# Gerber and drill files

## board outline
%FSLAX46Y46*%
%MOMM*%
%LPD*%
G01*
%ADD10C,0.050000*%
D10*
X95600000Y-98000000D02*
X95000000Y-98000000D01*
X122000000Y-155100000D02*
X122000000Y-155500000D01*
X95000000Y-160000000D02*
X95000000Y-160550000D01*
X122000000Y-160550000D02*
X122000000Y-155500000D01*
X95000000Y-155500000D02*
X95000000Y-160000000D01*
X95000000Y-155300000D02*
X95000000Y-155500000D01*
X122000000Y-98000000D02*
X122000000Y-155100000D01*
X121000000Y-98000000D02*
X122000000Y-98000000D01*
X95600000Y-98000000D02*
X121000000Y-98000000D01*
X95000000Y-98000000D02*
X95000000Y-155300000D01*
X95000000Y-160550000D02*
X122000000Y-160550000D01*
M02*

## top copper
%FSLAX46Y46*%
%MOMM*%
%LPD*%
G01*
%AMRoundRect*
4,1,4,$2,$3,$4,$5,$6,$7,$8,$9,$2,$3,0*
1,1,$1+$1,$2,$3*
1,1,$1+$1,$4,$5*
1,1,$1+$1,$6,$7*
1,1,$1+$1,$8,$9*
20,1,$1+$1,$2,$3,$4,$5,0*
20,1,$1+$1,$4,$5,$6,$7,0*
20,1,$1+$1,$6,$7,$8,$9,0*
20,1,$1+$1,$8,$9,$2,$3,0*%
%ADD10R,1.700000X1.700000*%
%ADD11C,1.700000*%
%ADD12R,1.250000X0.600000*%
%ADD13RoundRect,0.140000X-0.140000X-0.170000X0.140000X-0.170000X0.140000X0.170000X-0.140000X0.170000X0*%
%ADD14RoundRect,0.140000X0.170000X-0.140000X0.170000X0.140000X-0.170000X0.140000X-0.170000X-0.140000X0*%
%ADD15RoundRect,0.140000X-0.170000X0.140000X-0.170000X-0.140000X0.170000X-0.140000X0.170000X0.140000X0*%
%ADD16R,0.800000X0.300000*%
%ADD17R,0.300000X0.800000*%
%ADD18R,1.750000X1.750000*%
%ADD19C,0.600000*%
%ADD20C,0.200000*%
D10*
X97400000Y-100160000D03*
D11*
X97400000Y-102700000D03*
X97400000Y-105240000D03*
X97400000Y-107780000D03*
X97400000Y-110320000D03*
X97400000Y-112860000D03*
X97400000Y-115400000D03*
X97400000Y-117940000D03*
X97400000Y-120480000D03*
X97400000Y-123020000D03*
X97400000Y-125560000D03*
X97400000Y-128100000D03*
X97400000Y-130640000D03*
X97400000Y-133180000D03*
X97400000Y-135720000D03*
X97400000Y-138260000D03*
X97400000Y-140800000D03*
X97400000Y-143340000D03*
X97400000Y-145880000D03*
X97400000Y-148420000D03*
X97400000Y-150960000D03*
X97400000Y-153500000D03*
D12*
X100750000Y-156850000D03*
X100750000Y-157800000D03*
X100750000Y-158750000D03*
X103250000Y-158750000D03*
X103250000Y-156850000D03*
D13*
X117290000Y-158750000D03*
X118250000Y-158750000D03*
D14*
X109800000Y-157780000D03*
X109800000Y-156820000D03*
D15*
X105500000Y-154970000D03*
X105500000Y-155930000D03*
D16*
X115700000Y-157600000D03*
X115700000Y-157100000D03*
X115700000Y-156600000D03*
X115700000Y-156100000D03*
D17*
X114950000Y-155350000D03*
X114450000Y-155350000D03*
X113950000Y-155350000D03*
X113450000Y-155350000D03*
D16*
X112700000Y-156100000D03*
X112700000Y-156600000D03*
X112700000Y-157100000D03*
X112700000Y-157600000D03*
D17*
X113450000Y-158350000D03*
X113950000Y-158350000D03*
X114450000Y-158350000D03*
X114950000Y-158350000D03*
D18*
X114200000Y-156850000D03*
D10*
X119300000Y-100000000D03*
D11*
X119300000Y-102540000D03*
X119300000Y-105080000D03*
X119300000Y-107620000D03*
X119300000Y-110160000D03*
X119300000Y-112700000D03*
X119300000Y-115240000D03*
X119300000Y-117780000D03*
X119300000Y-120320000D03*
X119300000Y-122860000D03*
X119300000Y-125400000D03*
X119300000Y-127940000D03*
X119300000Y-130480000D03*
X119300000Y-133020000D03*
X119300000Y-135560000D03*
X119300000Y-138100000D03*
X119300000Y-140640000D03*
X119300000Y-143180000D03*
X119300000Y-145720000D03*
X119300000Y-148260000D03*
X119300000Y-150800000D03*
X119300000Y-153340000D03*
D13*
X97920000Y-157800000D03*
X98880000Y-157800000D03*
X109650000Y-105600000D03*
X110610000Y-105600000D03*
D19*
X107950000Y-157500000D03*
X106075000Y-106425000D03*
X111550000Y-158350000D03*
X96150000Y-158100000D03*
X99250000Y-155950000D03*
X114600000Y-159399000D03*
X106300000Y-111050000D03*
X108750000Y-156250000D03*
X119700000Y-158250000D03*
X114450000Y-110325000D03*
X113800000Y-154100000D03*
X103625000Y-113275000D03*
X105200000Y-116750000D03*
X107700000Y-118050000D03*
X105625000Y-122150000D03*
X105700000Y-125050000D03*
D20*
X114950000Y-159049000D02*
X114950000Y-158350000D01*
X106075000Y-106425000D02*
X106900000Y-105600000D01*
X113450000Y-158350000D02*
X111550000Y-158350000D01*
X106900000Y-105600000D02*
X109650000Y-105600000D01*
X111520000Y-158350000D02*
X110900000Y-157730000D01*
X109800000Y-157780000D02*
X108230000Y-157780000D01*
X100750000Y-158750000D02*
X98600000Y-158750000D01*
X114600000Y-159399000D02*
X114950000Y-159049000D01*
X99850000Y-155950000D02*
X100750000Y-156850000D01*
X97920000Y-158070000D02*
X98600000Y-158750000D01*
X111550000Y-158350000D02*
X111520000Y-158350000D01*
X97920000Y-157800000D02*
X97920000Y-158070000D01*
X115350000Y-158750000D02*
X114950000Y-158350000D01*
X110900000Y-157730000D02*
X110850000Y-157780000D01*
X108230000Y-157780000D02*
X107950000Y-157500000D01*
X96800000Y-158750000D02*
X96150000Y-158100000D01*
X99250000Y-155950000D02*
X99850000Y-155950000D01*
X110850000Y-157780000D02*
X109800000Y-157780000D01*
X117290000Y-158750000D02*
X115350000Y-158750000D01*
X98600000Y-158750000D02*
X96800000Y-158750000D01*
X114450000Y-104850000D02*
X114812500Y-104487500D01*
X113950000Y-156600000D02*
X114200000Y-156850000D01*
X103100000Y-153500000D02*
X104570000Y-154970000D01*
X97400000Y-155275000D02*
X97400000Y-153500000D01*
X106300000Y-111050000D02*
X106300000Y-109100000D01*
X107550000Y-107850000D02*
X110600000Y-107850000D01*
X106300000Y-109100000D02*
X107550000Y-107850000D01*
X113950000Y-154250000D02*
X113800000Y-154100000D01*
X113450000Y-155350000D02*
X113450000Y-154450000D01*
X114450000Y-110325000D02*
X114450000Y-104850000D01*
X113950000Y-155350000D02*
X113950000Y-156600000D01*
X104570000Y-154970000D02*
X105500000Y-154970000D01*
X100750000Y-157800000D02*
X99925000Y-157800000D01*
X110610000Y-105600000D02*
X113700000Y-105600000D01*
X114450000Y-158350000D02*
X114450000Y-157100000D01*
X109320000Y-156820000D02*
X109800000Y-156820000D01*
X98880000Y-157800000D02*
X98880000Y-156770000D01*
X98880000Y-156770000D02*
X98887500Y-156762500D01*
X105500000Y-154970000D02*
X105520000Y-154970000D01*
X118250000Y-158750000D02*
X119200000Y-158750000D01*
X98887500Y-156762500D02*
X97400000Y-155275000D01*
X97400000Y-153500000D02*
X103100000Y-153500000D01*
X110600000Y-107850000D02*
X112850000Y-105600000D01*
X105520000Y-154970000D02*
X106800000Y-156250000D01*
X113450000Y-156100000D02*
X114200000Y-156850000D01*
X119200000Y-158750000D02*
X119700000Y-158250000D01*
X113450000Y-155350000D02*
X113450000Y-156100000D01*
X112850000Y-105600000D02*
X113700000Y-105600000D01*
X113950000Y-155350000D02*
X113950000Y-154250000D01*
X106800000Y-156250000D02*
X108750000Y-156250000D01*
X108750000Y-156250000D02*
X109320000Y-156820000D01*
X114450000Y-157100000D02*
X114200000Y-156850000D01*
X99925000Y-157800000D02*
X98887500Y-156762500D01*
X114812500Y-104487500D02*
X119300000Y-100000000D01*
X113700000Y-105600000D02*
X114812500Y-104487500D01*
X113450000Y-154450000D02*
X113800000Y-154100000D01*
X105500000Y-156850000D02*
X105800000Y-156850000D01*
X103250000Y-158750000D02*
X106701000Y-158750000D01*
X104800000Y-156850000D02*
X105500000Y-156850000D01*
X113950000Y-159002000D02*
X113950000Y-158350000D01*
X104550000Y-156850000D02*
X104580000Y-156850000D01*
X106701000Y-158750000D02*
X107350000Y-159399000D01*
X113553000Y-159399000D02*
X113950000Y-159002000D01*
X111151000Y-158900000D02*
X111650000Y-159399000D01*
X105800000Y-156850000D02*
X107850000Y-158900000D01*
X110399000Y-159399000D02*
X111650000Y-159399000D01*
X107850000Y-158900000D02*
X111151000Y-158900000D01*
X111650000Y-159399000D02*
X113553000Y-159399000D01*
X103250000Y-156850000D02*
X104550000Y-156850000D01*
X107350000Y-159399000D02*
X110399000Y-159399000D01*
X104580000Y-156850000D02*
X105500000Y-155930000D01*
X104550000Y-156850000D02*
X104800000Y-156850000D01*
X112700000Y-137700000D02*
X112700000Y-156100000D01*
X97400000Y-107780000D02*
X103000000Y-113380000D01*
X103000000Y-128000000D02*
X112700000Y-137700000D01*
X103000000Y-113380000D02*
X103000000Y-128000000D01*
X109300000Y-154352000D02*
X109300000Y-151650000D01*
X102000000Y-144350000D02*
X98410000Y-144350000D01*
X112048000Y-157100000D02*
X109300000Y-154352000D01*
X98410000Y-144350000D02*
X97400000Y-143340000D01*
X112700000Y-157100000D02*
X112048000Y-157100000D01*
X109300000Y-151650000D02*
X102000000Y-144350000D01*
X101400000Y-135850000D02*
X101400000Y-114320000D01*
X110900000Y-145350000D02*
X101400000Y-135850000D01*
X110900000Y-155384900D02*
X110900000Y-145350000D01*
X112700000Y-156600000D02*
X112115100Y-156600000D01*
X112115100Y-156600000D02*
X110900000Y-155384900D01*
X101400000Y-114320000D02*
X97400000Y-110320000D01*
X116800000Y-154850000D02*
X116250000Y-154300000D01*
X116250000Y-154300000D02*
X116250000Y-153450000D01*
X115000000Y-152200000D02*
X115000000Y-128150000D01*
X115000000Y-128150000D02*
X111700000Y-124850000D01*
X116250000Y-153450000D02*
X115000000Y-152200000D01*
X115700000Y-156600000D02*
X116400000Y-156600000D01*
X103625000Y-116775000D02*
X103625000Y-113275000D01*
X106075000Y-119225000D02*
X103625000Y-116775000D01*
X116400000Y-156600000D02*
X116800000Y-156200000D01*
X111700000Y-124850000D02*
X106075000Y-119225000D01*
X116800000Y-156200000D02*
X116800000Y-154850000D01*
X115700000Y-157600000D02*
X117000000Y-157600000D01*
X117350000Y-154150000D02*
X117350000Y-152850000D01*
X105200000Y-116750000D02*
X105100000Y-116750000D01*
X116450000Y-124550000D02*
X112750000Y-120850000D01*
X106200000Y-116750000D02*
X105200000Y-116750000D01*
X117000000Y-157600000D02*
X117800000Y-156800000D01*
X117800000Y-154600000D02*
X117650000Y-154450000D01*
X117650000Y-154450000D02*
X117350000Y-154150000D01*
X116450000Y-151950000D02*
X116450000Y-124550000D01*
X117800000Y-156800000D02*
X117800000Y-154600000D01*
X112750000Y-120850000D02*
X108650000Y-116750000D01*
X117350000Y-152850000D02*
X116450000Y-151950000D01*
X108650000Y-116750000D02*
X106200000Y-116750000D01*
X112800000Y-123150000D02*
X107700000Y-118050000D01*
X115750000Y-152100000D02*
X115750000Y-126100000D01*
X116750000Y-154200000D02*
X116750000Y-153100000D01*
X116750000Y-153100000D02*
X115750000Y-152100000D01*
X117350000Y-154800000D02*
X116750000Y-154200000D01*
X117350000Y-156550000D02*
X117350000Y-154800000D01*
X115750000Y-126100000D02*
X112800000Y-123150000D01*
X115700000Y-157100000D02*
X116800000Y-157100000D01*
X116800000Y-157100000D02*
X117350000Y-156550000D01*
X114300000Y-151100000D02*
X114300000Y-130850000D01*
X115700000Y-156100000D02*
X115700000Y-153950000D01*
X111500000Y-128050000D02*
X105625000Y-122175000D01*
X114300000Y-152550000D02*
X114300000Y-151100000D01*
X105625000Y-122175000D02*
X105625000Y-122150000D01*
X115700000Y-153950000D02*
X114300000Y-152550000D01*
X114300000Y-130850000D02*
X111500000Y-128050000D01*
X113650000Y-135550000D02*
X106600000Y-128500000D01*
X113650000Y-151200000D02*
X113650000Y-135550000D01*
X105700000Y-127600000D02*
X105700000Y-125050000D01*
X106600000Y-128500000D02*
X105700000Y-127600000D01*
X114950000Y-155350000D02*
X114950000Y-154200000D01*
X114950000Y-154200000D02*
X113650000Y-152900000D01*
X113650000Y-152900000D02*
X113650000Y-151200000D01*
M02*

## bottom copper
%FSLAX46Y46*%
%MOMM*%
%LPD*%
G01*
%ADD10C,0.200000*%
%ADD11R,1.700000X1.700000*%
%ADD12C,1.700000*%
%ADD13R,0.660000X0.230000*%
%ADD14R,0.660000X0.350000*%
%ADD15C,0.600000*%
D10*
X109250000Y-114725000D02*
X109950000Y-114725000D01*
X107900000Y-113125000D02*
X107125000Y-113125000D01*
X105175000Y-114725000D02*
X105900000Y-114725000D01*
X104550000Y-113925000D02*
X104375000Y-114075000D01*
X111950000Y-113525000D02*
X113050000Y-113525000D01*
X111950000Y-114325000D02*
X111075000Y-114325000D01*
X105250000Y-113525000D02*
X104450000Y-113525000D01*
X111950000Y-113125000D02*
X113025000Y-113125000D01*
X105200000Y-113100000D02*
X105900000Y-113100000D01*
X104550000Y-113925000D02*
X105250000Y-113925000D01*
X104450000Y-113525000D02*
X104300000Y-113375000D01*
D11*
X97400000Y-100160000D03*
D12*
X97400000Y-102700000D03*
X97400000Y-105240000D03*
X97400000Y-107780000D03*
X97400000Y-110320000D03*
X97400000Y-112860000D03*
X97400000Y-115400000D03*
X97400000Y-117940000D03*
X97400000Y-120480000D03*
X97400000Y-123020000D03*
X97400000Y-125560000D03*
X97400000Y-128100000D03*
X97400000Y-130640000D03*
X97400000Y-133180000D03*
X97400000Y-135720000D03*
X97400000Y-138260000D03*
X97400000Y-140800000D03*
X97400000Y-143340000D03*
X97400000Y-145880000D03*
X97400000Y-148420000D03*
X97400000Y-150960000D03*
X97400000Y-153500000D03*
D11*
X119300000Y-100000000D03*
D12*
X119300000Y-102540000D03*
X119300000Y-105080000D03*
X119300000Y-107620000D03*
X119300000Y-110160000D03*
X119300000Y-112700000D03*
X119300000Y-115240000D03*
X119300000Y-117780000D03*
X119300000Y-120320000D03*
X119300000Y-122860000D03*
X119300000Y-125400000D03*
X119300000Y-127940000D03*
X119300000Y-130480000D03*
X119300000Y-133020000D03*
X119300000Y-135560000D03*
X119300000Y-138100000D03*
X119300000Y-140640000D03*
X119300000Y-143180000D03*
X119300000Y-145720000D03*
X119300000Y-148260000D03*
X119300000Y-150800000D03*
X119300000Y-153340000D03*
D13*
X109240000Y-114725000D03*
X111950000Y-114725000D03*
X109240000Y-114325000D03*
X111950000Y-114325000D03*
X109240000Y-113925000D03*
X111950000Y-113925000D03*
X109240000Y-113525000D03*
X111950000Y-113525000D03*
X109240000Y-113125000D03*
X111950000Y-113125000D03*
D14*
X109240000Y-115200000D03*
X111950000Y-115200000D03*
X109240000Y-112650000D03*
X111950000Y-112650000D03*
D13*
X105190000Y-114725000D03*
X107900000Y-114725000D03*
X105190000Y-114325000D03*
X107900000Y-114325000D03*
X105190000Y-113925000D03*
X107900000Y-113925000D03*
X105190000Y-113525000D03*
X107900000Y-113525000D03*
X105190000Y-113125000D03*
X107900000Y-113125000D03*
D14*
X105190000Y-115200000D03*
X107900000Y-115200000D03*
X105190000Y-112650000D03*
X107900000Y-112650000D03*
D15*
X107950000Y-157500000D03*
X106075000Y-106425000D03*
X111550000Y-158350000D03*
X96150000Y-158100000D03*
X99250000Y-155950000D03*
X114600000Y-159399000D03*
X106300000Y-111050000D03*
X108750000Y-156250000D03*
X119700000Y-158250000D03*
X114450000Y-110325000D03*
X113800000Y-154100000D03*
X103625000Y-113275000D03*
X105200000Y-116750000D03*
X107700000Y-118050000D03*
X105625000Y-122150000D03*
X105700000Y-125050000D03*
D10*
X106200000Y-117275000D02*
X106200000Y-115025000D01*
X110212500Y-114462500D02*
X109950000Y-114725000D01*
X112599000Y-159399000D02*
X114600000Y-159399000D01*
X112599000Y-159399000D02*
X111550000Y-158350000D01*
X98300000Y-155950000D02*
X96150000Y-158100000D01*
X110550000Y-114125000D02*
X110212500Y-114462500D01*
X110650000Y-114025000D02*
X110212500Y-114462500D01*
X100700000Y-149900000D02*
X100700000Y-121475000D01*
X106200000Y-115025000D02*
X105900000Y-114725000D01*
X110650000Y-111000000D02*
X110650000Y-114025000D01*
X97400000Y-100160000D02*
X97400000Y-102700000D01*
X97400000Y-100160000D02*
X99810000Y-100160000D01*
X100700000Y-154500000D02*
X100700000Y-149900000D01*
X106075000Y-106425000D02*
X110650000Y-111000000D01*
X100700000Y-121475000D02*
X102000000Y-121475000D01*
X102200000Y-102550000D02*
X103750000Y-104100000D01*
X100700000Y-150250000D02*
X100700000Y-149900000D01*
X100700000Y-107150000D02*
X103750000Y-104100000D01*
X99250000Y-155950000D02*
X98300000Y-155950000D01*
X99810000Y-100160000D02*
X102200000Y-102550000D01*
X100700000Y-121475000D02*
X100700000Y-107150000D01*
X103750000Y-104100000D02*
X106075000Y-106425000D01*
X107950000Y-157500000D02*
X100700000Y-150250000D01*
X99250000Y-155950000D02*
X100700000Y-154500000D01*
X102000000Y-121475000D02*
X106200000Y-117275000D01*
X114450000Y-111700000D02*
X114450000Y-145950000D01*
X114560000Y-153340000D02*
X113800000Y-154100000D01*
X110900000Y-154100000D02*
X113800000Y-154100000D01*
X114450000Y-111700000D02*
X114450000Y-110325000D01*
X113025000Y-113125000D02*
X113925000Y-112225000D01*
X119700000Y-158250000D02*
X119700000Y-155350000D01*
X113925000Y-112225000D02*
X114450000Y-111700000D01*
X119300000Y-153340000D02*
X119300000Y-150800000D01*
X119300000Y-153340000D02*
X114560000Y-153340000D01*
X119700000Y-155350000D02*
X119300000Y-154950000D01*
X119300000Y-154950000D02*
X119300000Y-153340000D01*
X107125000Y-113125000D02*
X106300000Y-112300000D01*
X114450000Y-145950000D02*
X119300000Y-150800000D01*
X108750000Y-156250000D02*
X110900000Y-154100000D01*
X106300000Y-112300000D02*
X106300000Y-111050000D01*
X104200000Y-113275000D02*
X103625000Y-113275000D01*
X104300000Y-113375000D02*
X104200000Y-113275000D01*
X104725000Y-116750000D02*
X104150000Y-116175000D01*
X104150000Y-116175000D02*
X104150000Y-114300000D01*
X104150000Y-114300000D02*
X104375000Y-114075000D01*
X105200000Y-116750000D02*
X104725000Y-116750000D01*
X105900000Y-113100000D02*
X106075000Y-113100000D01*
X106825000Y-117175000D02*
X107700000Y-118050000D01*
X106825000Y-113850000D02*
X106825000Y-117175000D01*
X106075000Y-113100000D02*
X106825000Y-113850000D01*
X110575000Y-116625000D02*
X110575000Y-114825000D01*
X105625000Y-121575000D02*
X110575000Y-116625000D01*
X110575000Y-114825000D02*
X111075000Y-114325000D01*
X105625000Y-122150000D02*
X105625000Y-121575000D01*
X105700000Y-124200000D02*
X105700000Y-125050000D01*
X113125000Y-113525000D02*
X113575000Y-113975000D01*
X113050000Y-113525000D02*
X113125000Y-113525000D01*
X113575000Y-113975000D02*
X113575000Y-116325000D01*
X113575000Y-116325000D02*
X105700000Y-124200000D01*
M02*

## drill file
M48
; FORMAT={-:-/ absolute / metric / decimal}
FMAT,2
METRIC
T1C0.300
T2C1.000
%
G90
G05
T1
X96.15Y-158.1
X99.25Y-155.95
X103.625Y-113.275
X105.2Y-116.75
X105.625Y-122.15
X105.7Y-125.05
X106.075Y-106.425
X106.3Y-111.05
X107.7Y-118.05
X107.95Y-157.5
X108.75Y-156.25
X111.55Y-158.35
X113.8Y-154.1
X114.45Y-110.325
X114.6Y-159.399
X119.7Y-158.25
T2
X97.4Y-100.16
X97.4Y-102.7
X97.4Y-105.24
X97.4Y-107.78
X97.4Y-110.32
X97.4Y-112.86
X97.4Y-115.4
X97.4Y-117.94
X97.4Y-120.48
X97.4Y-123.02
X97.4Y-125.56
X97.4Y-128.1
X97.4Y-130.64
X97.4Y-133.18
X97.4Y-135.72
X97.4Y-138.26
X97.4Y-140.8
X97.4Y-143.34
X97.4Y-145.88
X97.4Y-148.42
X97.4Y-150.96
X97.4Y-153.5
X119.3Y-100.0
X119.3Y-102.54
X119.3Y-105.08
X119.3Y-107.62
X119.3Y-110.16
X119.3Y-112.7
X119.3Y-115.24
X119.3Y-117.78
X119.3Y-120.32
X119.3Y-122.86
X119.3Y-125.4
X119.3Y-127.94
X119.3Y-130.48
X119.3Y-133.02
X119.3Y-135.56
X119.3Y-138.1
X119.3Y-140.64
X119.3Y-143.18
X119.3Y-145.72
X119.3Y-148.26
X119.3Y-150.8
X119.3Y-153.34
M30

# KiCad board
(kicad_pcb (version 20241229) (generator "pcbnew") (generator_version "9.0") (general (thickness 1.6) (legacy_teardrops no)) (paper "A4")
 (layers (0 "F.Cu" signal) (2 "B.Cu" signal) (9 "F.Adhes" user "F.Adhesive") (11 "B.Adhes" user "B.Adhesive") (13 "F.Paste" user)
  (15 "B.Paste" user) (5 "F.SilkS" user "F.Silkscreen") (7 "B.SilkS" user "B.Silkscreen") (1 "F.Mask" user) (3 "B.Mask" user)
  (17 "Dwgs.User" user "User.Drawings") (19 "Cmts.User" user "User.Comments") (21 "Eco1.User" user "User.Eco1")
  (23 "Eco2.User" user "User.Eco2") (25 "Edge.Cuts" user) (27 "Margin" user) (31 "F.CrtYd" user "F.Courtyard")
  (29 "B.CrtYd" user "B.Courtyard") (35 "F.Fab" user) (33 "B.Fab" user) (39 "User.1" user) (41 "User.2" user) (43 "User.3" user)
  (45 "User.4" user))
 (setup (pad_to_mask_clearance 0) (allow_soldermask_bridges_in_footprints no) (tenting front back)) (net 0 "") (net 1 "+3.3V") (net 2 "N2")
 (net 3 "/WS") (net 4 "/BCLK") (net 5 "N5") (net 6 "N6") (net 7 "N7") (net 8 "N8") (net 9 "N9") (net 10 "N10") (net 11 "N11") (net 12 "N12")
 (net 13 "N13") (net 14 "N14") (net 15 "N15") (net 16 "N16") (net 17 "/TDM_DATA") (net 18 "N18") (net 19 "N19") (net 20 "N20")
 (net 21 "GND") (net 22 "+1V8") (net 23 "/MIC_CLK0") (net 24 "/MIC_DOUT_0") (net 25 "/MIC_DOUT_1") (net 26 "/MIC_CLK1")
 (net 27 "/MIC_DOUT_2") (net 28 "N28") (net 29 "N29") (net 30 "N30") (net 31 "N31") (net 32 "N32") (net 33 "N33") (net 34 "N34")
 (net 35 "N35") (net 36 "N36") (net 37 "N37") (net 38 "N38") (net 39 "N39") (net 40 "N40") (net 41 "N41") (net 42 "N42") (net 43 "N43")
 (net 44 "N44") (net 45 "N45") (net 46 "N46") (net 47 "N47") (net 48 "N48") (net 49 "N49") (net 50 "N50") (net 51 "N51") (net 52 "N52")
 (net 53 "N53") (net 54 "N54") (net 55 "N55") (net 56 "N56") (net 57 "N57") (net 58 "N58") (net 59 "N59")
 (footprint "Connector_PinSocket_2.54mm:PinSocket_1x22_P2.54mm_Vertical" (layer "F.Cu") (at 97.4 100.16)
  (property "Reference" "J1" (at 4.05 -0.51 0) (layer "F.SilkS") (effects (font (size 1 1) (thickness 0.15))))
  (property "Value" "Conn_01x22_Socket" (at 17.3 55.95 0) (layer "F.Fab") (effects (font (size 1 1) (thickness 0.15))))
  (pad "1" thru_hole rect (at 0 0) (size 1.7 1.7) (drill 1) (layers "*.Cu" "*.Mask") (remove_unused_layers no) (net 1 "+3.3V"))
  (pad "2" thru_hole circle (at 0 2.54) (size 1.7 1.7) (drill 1) (layers "*.Cu" "*.Mask") (remove_unused_layers no) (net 1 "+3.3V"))
  (pad "3" thru_hole circle (at 0 5.08) (size 1.7 1.7) (drill 1) (layers "*.Cu" "*.Mask") (remove_unused_layers no) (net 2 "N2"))
  (pad "4" thru_hole circle (at 0 7.62) (size 1.7 1.7) (drill 1) (layers "*.Cu" "*.Mask") (remove_unused_layers no) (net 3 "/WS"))
  (pad "5" thru_hole circle (at 0 10.16) (size 1.7 1.7) (drill 1) (layers "*.Cu" "*.Mask") (remove_unused_layers no) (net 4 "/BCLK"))
  (pad "6" thru_hole circle (at 0 12.7) (size 1.7 1.7) (drill 1) (layers "*.Cu" "*.Mask") (remove_unused_layers no) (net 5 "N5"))
  (pad "7" thru_hole circle (at 0 15.24) (size 1.7 1.7) (drill 1) (layers "*.Cu" "*.Mask") (remove_unused_layers no) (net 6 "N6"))
  (pad "8" thru_hole circle (at 0 17.78) (size 1.7 1.7) (drill 1) (layers "*.Cu" "*.Mask") (remove_unused_layers no) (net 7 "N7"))
  (pad "9" thru_hole circle (at 0 20.32) (size 1.7 1.7) (drill 1) (layers "*.Cu" "*.Mask") (remove_unused_layers no) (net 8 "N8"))
  (pad "10" thru_hole circle (at 0 22.86) (size 1.7 1.7) (drill 1) (layers "*.Cu" "*.Mask") (remove_unused_layers no) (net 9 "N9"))
  (pad "11" thru_hole circle (at 0 25.4) (size 1.7 1.7) (drill 1) (layers "*.Cu" "*.Mask") (remove_unused_layers no) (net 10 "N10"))
  (pad "12" thru_hole circle (at 0 27.94) (size 1.7 1.7) (drill 1) (layers "*.Cu" "*.Mask") (remove_unused_layers no) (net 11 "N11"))
  (pad "13" thru_hole circle (at 0 30.48) (size 1.7 1.7) (drill 1) (layers "*.Cu" "*.Mask") (remove_unused_layers no) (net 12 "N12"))
  (pad "14" thru_hole circle (at 0 33.02) (size 1.7 1.7) (drill 1) (layers "*.Cu" "*.Mask") (remove_unused_layers no) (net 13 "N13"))
  (pad "15" thru_hole circle (at 0 35.56) (size 1.7 1.7) (drill 1) (layers "*.Cu" "*.Mask") (remove_unused_layers no) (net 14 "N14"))
  (pad "16" thru_hole circle (at 0 38.1) (size 1.7 1.7) (drill 1) (layers "*.Cu" "*.Mask") (remove_unused_layers no) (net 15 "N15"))
  (pad "17" thru_hole circle (at 0 40.64) (size 1.7 1.7) (drill 1) (layers "*.Cu" "*.Mask") (remove_unused_layers no) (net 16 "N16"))
  (pad "18" thru_hole circle (at 0 43.18) (size 1.7 1.7) (drill 1) (layers "*.Cu" "*.Mask") (remove_unused_layers no) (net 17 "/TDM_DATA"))
  (pad "19" thru_hole circle (at 0 45.72) (size 1.7 1.7) (drill 1) (layers "*.Cu" "*.Mask") (remove_unused_layers no) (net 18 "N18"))
  (pad "20" thru_hole circle (at 0 48.26) (size 1.7 1.7) (drill 1) (layers "*.Cu" "*.Mask") (remove_unused_layers no) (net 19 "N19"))
  (pad "21" thru_hole circle (at 0 50.8) (size 1.7 1.7) (drill 1) (layers "*.Cu" "*.Mask") (remove_unused_layers no) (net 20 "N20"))
  (pad "22" thru_hole circle (at 0 53.34) (size 1.7 1.7) (drill 1) (layers "*.Cu" "*.Mask") (remove_unused_layers no) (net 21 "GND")))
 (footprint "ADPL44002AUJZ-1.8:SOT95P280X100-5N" (layer "F.Cu") (at 102 157.8)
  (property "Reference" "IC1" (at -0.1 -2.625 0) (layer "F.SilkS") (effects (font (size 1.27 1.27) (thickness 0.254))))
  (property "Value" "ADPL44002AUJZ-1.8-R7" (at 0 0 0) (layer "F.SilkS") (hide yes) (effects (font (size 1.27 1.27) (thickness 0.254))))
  (pad "1" smd rect (at -1.25 -0.95 90) (size 0.6 1.25) (layers "F.Cu" "F.Mask" "F.Paste") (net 1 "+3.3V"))
  (pad "2" smd rect (at -1.25 0 90) (size 0.6 1.25) (layers "F.Cu" "F.Mask" "F.Paste") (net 21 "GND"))
  (pad "3" smd rect (at -1.25 0.95 90) (size 0.6 1.25) (layers "F.Cu" "F.Mask" "F.Paste") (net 1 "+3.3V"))
  (pad "4" smd rect (at 1.25 0.95 90) (size 0.6 1.25) (layers "F.Cu" "F.Mask" "F.Paste") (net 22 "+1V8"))
  (pad "5" smd rect (at 1.25 -0.95 90) (size 0.6 1.25) (layers "F.Cu" "F.Mask" "F.Paste") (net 22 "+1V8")))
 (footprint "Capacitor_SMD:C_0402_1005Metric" (layer "F.Cu") (at 117.77 158.75)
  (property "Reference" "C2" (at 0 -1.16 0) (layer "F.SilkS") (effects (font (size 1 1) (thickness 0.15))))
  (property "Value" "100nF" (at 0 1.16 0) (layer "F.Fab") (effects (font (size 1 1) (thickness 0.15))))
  (pad "1" smd roundrect (at -0.48 0) (size 0.56 0.62) (layers "F.Cu" "F.Mask" "F.Paste") (roundrect_rratio 0.25) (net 1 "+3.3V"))
  (pad "2" smd roundrect (at 0.48 0) (size 0.56 0.62) (layers "F.Cu" "F.Mask" "F.Paste") (roundrect_rratio 0.25) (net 21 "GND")))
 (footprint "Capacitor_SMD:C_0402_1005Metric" (layer "F.Cu") (at 109.8 157.3 90)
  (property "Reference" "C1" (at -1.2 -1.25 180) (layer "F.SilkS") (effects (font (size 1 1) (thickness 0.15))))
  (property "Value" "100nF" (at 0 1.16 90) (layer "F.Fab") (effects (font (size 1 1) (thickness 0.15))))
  (pad "1" smd roundrect (at -0.48 0 90) (size 0.56 0.62) (layers "F.Cu" "F.Mask" "F.Paste") (roundrect_rratio 0.25) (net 1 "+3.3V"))
  (pad "2" smd roundrect (at 0.48 0 90) (size 0.56 0.62) (layers "F.Cu" "F.Mask" "F.Paste") (roundrect_rratio 0.25) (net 21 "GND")))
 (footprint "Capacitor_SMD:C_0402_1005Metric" (layer "F.Cu") (at 105.5 155.45 -90)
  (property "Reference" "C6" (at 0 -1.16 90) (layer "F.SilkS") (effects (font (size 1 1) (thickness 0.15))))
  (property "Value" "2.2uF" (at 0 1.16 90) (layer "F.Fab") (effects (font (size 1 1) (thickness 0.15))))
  (pad "1" smd roundrect (at -0.48 0 270) (size 0.56 0.62) (layers "F.Cu" "F.Mask" "F.Paste") (roundrect_rratio 0.25) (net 21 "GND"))
  (pad "2" smd roundrect (at 0.48 0 270) (size 0.56 0.62) (layers "F.Cu" "F.Mask" "F.Paste") (roundrect_rratio 0.25) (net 22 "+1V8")))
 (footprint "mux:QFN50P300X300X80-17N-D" (layer "F.Cu") (at 114.2 156.85 180)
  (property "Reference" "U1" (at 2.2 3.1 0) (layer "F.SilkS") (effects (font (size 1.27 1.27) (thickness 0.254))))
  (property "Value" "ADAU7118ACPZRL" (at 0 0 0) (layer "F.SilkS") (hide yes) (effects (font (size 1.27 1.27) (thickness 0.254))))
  (pad "1" smd rect (at -1.5 -0.75 270) (size 0.3 0.8) (layers "F.Cu" "F.Mask" "F.Paste") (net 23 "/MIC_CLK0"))
  (pad "2" smd rect (at -1.5 -0.25 270) (size 0.3 0.8) (layers "F.Cu" "F.Mask" "F.Paste") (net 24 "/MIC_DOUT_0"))
  (pad "3" smd rect (at -1.5 0.25 270) (size 0.3 0.8) (layers "F.Cu" "F.Mask" "F.Paste") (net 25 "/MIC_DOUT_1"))
  (pad "4" smd rect (at -1.5 0.75 270) (size 0.3 0.8) (layers "F.Cu" "F.Mask" "F.Paste") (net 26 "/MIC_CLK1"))
  (pad "5" smd rect (at -0.75 1.5 180) (size 0.3 0.8) (layers "F.Cu" "F.Mask" "F.Paste") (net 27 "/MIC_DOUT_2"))
  (pad "6" smd rect (at -0.25 1.5 180) (size 0.3 0.8) (layers "F.Cu" "F.Mask" "F.Paste") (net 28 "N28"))
  (pad "7" smd rect (at 0.25 1.5 180) (size 0.3 0.8) (layers "F.Cu" "F.Mask" "F.Paste") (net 21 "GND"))
  (pad "8" smd rect (at 0.75 1.5 180) (size 0.3 0.8) (layers "F.Cu" "F.Mask" "F.Paste") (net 21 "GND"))
  (pad "9" smd rect (at 1.5 0.75 270) (size 0.3 0.8) (layers "F.Cu" "F.Mask" "F.Paste") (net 3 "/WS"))
  (pad "10" smd rect (at 1.5 0.25 270) (size 0.3 0.8) (layers "F.Cu" "F.Mask" "F.Paste") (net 4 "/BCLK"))
  (pad "11" smd rect (at 1.5 -0.25 270) (size 0.3 0.8) (layers "F.Cu" "F.Mask" "F.Paste") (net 17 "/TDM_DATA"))
  (pad "12" smd rect (at 1.5 -0.75 270) (size 0.3 0.8) (layers "F.Cu" "F.Mask" "F.Paste") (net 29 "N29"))
  (pad "13" smd rect (at 0.75 -1.5 180) (size 0.3 0.8) (layers "F.Cu" "F.Mask" "F.Paste") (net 1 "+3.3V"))
  (pad "14" smd rect (at 0.25 -1.5 180) (size 0.3 0.8) (layers "F.Cu" "F.Mask" "F.Paste") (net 22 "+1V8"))
  (pad "15" smd rect (at -0.25 -1.5 180) (size 0.3 0.8) (layers "F.Cu" "F.Mask" "F.Paste") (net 21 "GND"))
  (pad "16" smd rect (at -0.75 -1.5 180) (size 0.3 0.8) (layers "F.Cu" "F.Mask" "F.Paste") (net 1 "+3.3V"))
  (pad "17" smd rect (at 0 0 180) (size 1.75 1.75) (layers "F.Cu" "F.Mask" "F.Paste") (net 21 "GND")))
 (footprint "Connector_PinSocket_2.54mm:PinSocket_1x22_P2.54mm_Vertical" (layer "F.Cu") (at 119.3 100)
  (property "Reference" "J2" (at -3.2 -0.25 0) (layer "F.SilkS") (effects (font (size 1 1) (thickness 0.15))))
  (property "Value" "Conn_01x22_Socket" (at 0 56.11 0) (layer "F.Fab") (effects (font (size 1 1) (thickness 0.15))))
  (pad "1" thru_hole rect (at 0 0) (size 1.7 1.7) (drill 1) (layers "*.Cu" "*.Mask") (remove_unused_layers no) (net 21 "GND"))
  (pad "2" thru_hole circle (at 0 2.54) (size 1.7 1.7) (drill 1) (layers "*.Cu" "*.Mask") (remove_unused_layers no) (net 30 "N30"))
  (pad "3" thru_hole circle (at 0 5.08) (size 1.7 1.7) (drill 1) (layers "*.Cu" "*.Mask") (remove_unused_layers no) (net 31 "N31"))
  (pad "4" thru_hole circle (at 0 7.62) (size 1.7 1.7) (drill 1) (layers "*.Cu" "*.Mask") (remove_unused_layers no) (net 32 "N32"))
  (pad "5" thru_hole circle (at 0 10.16) (size 1.7 1.7) (drill 1) (layers "*.Cu" "*.Mask") (remove_unused_layers no) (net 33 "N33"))
  (pad "6" thru_hole circle (at 0 12.7) (size 1.7 1.7) (drill 1) (layers "*.Cu" "*.Mask") (remove_unused_layers no) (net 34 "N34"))
  (pad "7" thru_hole circle (at 0 15.24) (size 1.7 1.7) (drill 1) (layers "*.Cu" "*.Mask") (remove_unused_layers no) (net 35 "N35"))
  (pad "8" thru_hole circle (at 0 17.78) (size 1.7 1.7) (drill 1) (layers "*.Cu" "*.Mask") (remove_unused_layers no) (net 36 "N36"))
  (pad "9" thru_hole circle (at 0 20.32) (size 1.7 1.7) (drill 1) (layers "*.Cu" "*.Mask") (remove_unused_layers no) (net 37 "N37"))
  (pad "10" thru_hole circle (at 0 22.86) (size 1.7 1.7) (drill 1) (layers "*.Cu" "*.Mask") (remove_unused_layers no) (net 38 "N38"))
  (pad "11" thru_hole circle (at 0 25.4) (size 1.7 1.7) (drill 1) (layers "*.Cu" "*.Mask") (remove_unused_layers no) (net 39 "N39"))
  (pad "12" thru_hole circle (at 0 27.94) (size 1.7 1.7) (drill 1) (layers "*.Cu" "*.Mask") (remove_unused_layers no) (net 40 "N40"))
  (pad "13" thru_hole circle (at 0 30.48) (size 1.7 1.7) (drill 1) (layers "*.Cu" "*.Mask") (remove_unused_layers no) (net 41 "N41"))
  (pad "14" thru_hole circle (at 0 33.02) (size 1.7 1.7) (drill 1) (layers "*.Cu" "*.Mask") (remove_unused_layers no) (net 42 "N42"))
  (pad "15" thru_hole circle (at 0 35.56) (size 1.7 1.7) (drill 1) (layers "*.Cu" "*.Mask") (remove_unused_layers no) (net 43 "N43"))
  (pad "16" thru_hole circle (at 0 38.1) (size 1.7 1.7) (drill 1) (layers "*.Cu" "*.Mask") (remove_unused_layers no) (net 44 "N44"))
  (pad "17" thru_hole circle (at 0 40.64) (size 1.7 1.7) (drill 1) (layers "*.Cu" "*.Mask") (remove_unused_layers no) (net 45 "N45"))
  (pad "18" thru_hole circle (at 0 43.18) (size 1.7 1.7) (drill 1) (layers "*.Cu" "*.Mask") (remove_unused_layers no) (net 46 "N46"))
  (pad "19" thru_hole circle (at 0 45.72) (size 1.7 1.7) (drill 1) (layers "*.Cu" "*.Mask") (remove_unused_layers no) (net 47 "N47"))
  (pad "20" thru_hole circle (at 0 48.26) (size 1.7 1.7) (drill 1) (layers "*.Cu" "*.Mask") (remove_unused_layers no) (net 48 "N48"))
  (pad "21" thru_hole circle (at 0 50.8) (size 1.7 1.7) (drill 1) (layers "*.Cu" "*.Mask") (remove_unused_layers no) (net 21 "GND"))
  (pad "22" thru_hole circle (at 0 53.34) (size 1.7 1.7) (drill 1) (layers "*.Cu" "*.Mask") (remove_unused_layers no) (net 21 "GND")))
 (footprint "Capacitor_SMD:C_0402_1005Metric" (layer "F.Cu") (at 98.4 157.8)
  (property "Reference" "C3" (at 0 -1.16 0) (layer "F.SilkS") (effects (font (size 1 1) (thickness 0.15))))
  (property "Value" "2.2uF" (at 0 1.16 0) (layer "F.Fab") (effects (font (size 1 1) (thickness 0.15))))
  (pad "1" smd roundrect (at -0.48 0) (size 0.56 0.62) (layers "F.Cu" "F.Mask" "F.Paste") (roundrect_rratio 0.25) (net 1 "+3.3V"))
  (pad "2" smd roundrect (at 0.48 0) (size 0.56 0.62) (layers "F.Cu" "F.Mask" "F.Paste") (roundrect_rratio 0.25) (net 21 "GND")))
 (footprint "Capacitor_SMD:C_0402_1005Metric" (layer "F.Cu") (at 110.13 105.6)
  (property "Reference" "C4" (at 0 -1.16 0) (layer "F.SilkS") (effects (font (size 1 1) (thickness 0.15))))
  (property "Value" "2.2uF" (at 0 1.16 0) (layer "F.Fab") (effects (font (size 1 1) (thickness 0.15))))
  (pad "1" smd roundrect (at -0.48 0) (size 0.56 0.62) (layers "F.Cu" "F.Mask" "F.Paste") (roundrect_rratio 0.25) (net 1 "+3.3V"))
  (pad "2" smd roundrect (at 0.48 0) (size 0.56 0.62) (layers "F.Cu" "F.Mask" "F.Paste") (roundrect_rratio 0.25) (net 21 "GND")))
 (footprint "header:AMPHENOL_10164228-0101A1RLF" (layer "B.Cu") (at 110.595 113.925 90)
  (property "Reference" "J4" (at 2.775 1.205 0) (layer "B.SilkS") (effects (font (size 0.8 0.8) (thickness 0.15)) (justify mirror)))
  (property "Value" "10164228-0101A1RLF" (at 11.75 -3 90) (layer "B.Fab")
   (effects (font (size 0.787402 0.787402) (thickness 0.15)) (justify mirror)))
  (pad "1" smd rect (at -0.8 -1.355 90) (size 0.23 0.66) (layers "B.Cu") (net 1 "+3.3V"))
  (pad "2" smd rect (at -0.8 1.355 90) (size 0.23 0.66) (layers "B.Cu") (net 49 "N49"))
  (pad "3" smd rect (at -0.4 -1.355 90) (size 0.23 0.66) (layers "B.Cu") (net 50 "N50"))
  (pad "4" smd rect (at -0.4 1.355 90) (size 0.23 0.66) (layers "B.Cu") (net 26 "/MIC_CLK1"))
  (pad "5" smd rect (at 0 -1.355 90) (size 0.23 0.66) (layers "B.Cu") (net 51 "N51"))
  (pad "6" smd rect (at 0 1.355 90) (size 0.23 0.66) (layers "B.Cu") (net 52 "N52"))
  (pad "7" smd rect (at 0.4 -1.355 90) (size 0.23 0.66) (layers "B.Cu") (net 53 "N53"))
  (pad "8" smd rect (at 0.4 1.355 90) (size 0.23 0.66) (layers "B.Cu") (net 27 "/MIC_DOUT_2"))
  (pad "9" smd rect (at 0.8 -1.355 90) (size 0.23 0.66) (layers "B.Cu") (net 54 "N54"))
  (pad "10" smd rect (at 0.8 1.355 90) (size 0.23 0.66) (layers "B.Cu") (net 21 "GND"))
  (pad "SH1" smd rect (at -1.275 -1.355 90) (size 0.35 0.66) (layers "B.Cu"))
  (pad "SH2" smd rect (at -1.275 1.355 90) (size 0.35 0.66) (layers "B.Cu"))
  (pad "SH3" smd rect (at 1.275 -1.355 90) (size 0.35 0.66) (layers "B.Cu"))
  (pad "SH4" smd rect (at 1.275 1.355 90) (size 0.35 0.66) (layers "B.Cu")))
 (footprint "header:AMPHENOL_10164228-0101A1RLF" (layer "B.Cu") (at 106.545 113.925 90)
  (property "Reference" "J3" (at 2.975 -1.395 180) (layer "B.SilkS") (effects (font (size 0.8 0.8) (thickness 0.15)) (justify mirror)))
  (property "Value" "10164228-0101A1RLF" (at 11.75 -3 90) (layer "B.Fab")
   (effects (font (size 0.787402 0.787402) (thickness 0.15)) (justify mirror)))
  (pad "1" smd rect (at -0.8 -1.355 90) (size 0.23 0.66) (layers "B.Cu") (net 1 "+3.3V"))
  (pad "2" smd rect (at -0.8 1.355 90) (size 0.23 0.66) (layers "B.Cu") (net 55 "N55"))
  (pad "3" smd rect (at -0.4 -1.355 90) (size 0.23 0.66) (layers "B.Cu") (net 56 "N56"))
  (pad "4" smd rect (at -0.4 1.355 90) (size 0.23 0.66) (layers "B.Cu") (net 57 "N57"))
  (pad "5" smd rect (at 0 -1.355 90) (size 0.23 0.66) (layers "B.Cu") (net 23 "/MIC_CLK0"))
  (pad "6" smd rect (at 0 1.355 90) (size 0.23 0.66) (layers "B.Cu") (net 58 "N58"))
  (pad "7" smd rect (at 0.4 -1.355 90) (size 0.23 0.66) (layers "B.Cu") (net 25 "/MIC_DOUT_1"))
  (pad "8" smd rect (at 0.4 1.355 90) (size 0.23 0.66) (layers "B.Cu") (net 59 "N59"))
  (pad "9" smd rect (at 0.8 -1.355 90) (size 0.23 0.66) (layers "B.Cu") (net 24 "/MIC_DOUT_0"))
  (pad "10" smd rect (at 0.8 1.355 90) (size 0.23 0.66) (layers "B.Cu") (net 21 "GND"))
  (pad "SH1" smd rect (at -1.275 -1.355 90) (size 0.35 0.66) (layers "B.Cu"))
  (pad "SH2" smd rect (at -1.275 1.355 90) (size 0.35 0.66) (layers "B.Cu"))
  (pad "SH3" smd rect (at 1.275 -1.355 90) (size 0.35 0.66) (layers "B.Cu"))
  (pad "SH4" smd rect (at 1.275 1.355 90) (size 0.35 0.66) (layers "B.Cu")))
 (gr_line (start 109.25 114.725) (end 109.95 114.725) (stroke (width 0.2) (type default)) (layer "B.Cu") (net 1))
 (gr_line (start 107.9 113.125) (end 107.125 113.125) (stroke (width 0.2) (type default)) (layer "B.Cu") (net 21))
 (gr_line (start 105.175 114.725) (end 105.9 114.725) (stroke (width 0.2) (type default)) (layer "B.Cu") (net 1))
 (gr_line (start 104.55 113.925) (end 104.375 114.075) (stroke (width 0.2) (type default)) (layer "B.Cu") (net 23))
 (gr_line (start 111.95 113.525) (end 113.05 113.525) (stroke (width 0.2) (type default)) (layer "B.Cu") (net 27))
 (gr_line (start 111.95 114.325) (end 111.075 114.325) (stroke (width 0.2) (type default)) (layer "B.Cu") (net 26))
 (gr_line (start 105.25 113.525) (end 104.45 113.525) (stroke (width 0.2) (type default)) (layer "B.Cu") (net 25))
 (gr_line (start 111.95 113.125) (end 113.025 113.125) (stroke (width 0.2) (type default)) (layer "B.Cu") (net 21))
 (gr_line (start 105.2 113.1) (end 105.9 113.1) (stroke (width 0.2) (type default)) (layer "B.Cu") (net 24))
 (gr_line (start 104.55 113.925) (end 105.25 113.925) (stroke (width 0.2) (type default)) (layer "B.Cu") (net 23))
 (gr_line (start 104.45 113.525) (end 104.3 113.375) (stroke (width 0.2) (type default)) (layer "B.Cu") (net 25))
 (gr_line (start 95.6 98) (end 95 98) (stroke (width 0.05) (type default)) (layer "Edge.Cuts"))
 (gr_line (start 122 155.1) (end 122 155.5) (stroke (width 0.05) (type default)) (layer "Edge.Cuts"))
 (gr_line (start 95 160) (end 95 160.55) (stroke (width 0.05) (type default)) (layer "Edge.Cuts"))
 (gr_line (start 122 160.55) (end 122 155.5) (stroke (width 0.05) (type default)) (layer "Edge.Cuts"))
 (gr_line (start 95 155.5) (end 95 160) (stroke (width 0.05) (type default)) (layer "Edge.Cuts"))
 (gr_line (start 95 155.3) (end 95 155.5) (stroke (width 0.05) (type default)) (layer "Edge.Cuts"))
 (gr_line (start 122 98) (end 122 155.1) (stroke (width 0.05) (type default)) (layer "Edge.Cuts"))
 (gr_line (start 121 98) (end 122 98) (stroke (width 0.05) (type default)) (layer "Edge.Cuts"))
 (gr_line (start 95.6 98) (end 121 98) (stroke (width 0.05) (type solid)) (layer "Edge.Cuts"))
 (gr_line (start 95 98) (end 95 155.3) (stroke (width 0.05) (type default)) (layer "Edge.Cuts"))
 (gr_line (start 95 160.55) (end 122 160.55) (stroke (width 0.05) (type default)) (layer "Edge.Cuts"))
 (segment (start 114.95 159.049) (end 114.95 158.35) (width 0.2) (layer "F.Cu") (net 1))
 (segment (start 106.075 106.425) (end 106.9 105.6) (width 0.2) (layer "F.Cu") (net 1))
 (segment (start 113.45 158.35) (end 111.55 158.35) (width 0.2) (layer "F.Cu") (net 1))
 (segment (start 106.9 105.6) (end 109.65 105.6) (width 0.2) (layer "F.Cu") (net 1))
 (segment (start 111.52 158.35) (end 110.9 157.73) (width 0.2) (layer "F.Cu") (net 1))
 (segment (start 109.8 157.78) (end 108.23 157.78) (width 0.2) (layer "F.Cu") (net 1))
 (segment (start 100.75 158.75) (end 98.6 158.75) (width 0.2) (layer "F.Cu") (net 1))
 (segment (start 114.6 159.399) (end 114.95 159.049) (width 0.2) (layer "F.Cu") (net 1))
 (segment (start 99.85 155.95) (end 100.75 156.85) (width 0.2) (layer "F.Cu") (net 1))
 (segment (start 97.92 158.07) (end 98.6 158.75) (width 0.2) (layer "F.Cu") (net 1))
 (segment (start 111.55 158.35) (end 111.52 158.35) (width 0.2) (layer "F.Cu") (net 1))
 (segment (start 97.92 157.8) (end 97.92 158.07) (width 0.2) (layer "F.Cu") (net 1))
 (segment (start 115.35 158.75) (end 114.95 158.35) (width 0.2) (layer "F.Cu") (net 1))
 (segment (start 110.9 157.73) (end 110.85 157.78) (width 0.2) (layer "F.Cu") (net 1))
 (segment (start 108.23 157.78) (end 107.95 157.5) (width 0.2) (layer "F.Cu") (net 1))
 (segment (start 96.8 158.75) (end 96.15 158.1) (width 0.2) (layer "F.Cu") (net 1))
 (segment (start 99.25 155.95) (end 99.85 155.95) (width 0.2) (layer "F.Cu") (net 1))
 (segment (start 110.85 157.78) (end 109.8 157.78) (width 0.2) (layer "F.Cu") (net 1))
 (segment (start 117.29 158.75) (end 115.35 158.75) (width 0.2) (layer "F.Cu") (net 1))
 (segment (start 98.6 158.75) (end 96.8 158.75) (width 0.2) (layer "F.Cu") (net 1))
 (via (at 107.95 157.5) (size 0.6) (drill 0.3) (layers "F.Cu" "B.Cu") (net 1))
 (via (at 106.075 106.425) (size 0.6) (drill 0.3) (layers "F.Cu" "B.Cu") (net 1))
 (via (at 111.55 158.35) (size 0.6) (drill 0.3) (layers "F.Cu" "B.Cu") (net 1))
 (via (at 96.15 158.1) (size 0.6) (drill 0.3) (layers "F.Cu" "B.Cu") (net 1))
 (via (at 99.25 155.95) (size 0.6) (drill 0.3) (layers "F.Cu" "B.Cu") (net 1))
 (via (at 114.6 159.399) (size 0.6) (drill 0.3) (layers "F.Cu" "B.Cu") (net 1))
 (segment (start 106.2 117.275) (end 106.2 115.025) (width 0.2) (layer "B.Cu") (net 1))
 (segment (start 110.2125 114.4625) (end 109.95 114.725) (width 0.2) (layer "B.Cu") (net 1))
 (segment (start 112.599 159.399) (end 114.6 159.399) (width 0.2) (layer "B.Cu") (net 1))
 (segment (start 112.599 159.399) (end 111.55 158.35) (width 0.2) (layer "B.Cu") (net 1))
 (segment (start 98.3 155.95) (end 96.15 158.1) (width 0.2) (layer "B.Cu") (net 1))
 (segment (start 110.55 114.125) (end 110.2125 114.4625) (width 0.2) (layer "B.Cu") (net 1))
 (segment (start 110.65 114.025) (end 110.2125 114.4625) (width 0.2) (layer "B.Cu") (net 1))
 (segment (start 100.7 149.9) (end 100.7 121.475) (width 0.2) (layer "B.Cu") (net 1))
 (segment (start 106.2 115.025) (end 105.9 114.725) (width 0.2) (layer "B.Cu") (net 1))
 (segment (start 110.65 111) (end 110.65 114.025) (width 0.2) (layer "B.Cu") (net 1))
 (segment (start 97.4 100.16) (end 97.4 102.7) (width 0.2) (layer "B.Cu") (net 1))
 (segment (start 97.4 100.16) (end 99.81 100.16) (width 0.2) (layer "B.Cu") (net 1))
 (segment (start 100.7 154.5) (end 100.7 149.9) (width 0.2) (layer "B.Cu") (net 1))
 (segment (start 106.075 106.425) (end 110.65 111) (width 0.2) (layer "B.Cu") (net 1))
 (segment (start 100.7 121.475) (end 102 121.475) (width 0.2) (layer "B.Cu") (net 1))
 (segment (start 102.2 102.55) (end 103.75 104.1) (width 0.2) (layer "B.Cu") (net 1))
 (segment (start 100.7 150.25) (end 100.7 149.9) (width 0.2) (layer "B.Cu") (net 1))
 (segment (start 100.7 107.15) (end 103.75 104.1) (width 0.2) (layer "B.Cu") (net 1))
 (segment (start 99.25 155.95) (end 98.3 155.95) (width 0.2) (layer "B.Cu") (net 1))
 (segment (start 99.81 100.16) (end 102.2 102.55) (width 0.2) (layer "B.Cu") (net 1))
 (segment (start 100.7 121.475) (end 100.7 107.15) (width 0.2) (layer "B.Cu") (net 1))
 (segment (start 103.75 104.1) (end 106.075 106.425) (width 0.2) (layer "B.Cu") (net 1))
 (segment (start 107.95 157.5) (end 100.7 150.25) (width 0.2) (layer "B.Cu") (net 1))
 (segment (start 99.25 155.95) (end 100.7 154.5) (width 0.2) (layer "B.Cu") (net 1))
 (segment (start 102 121.475) (end 106.2 117.275) (width 0.2) (layer "B.Cu") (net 1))
 (segment (start 114.45 104.85) (end 114.8125 104.4875) (width 0.2) (layer "F.Cu") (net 21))
 (segment (start 113.95 156.6) (end 114.2 156.85) (width 0.2) (layer "F.Cu") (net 21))
 (segment (start 103.1 153.5) (end 104.57 154.97) (width 0.2) (layer "F.Cu") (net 21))
 (segment (start 97.4 155.275) (end 97.4 153.5) (width 0.2) (layer "F.Cu") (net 21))
 (segment (start 106.3 111.05) (end 106.3 109.1) (width 0.2) (layer "F.Cu") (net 21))
 (segment (start 107.55 107.85) (end 110.6 107.85) (width 0.2) (layer "F.Cu") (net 21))
 (segment (start 106.3 109.1) (end 107.55 107.85) (width 0.2) (layer "F.Cu") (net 21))
 (segment (start 113.95 154.25) (end 113.8 154.1) (width 0.2) (layer "F.Cu") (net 21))
 (segment (start 113.45 155.35) (end 113.45 154.45) (width 0.2) (layer "F.Cu") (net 21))
 (segment (start 114.45 110.325) (end 114.45 104.85) (width 0.2) (layer "F.Cu") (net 21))
 (segment (start 113.95 155.35) (end 113.95 156.6) (width 0.2) (layer "F.Cu") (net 21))
 (segment (start 104.57 154.97) (end 105.5 154.97) (width 0.2) (layer "F.Cu") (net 21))
 (segment (start 100.75 157.8) (end 99.925 157.8) (width 0.2) (layer "F.Cu") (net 21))
 (segment (start 110.61 105.6) (end 113.7 105.6) (width 0.2) (layer "F.Cu") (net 21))
 (segment (start 114.45 158.35) (end 114.45 157.1) (width 0.2) (layer "F.Cu") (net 21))
 (segment (start 109.32 156.82) (end 109.8 156.82) (width 0.2) (layer "F.Cu") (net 21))
 (segment (start 98.88 157.8) (end 98.88 156.77) (width 0.2) (layer "F.Cu") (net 21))
 (segment (start 98.88 156.77) (end 98.8875 156.7625) (width 0.2) (layer "F.Cu") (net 21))
 (segment (start 105.5 154.97) (end 105.52 154.97) (width 0.2) (layer "F.Cu") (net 21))
 (segment (start 118.25 158.75) (end 119.2 158.75) (width 0.2) (layer "F.Cu") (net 21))
 (segment (start 98.8875 156.7625) (end 97.4 155.275) (width 0.2) (layer "F.Cu") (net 21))
 (segment (start 97.4 153.5) (end 103.1 153.5) (width 0.2) (layer "F.Cu") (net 21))
 (segment (start 110.6 107.85) (end 112.85 105.6) (width 0.2) (layer "F.Cu") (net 21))
 (segment (start 105.52 154.97) (end 106.8 156.25) (width 0.2) (layer "F.Cu") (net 21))
 (segment (start 113.45 156.1) (end 114.2 156.85) (width 0.2) (layer "F.Cu") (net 21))
 (segment (start 119.2 158.75) (end 119.7 158.25) (width 0.2) (layer "F.Cu") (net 21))
 (segment (start 113.45 155.35) (end 113.45 156.1) (width 0.2) (layer "F.Cu") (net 21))
 (segment (start 112.85 105.6) (end 113.7 105.6) (width 0.2) (layer "F.Cu") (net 21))
 (segment (start 113.95 155.35) (end 113.95 154.25) (width 0.2) (layer "F.Cu") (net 21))
 (segment (start 106.8 156.25) (end 108.75 156.25) (width 0.2) (layer "F.Cu") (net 21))
 (segment (start 108.75 156.25) (end 109.32 156.82) (width 0.2) (layer "F.Cu") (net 21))
 (segment (start 114.45 157.1) (end 114.2 156.85) (width 0.2) (layer "F.Cu") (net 21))
 (segment (start 99.925 157.8) (end 98.8875 156.7625) (width 0.2) (layer "F.Cu") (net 21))
 (segment (start 114.8125 104.4875) (end 119.3 100) (width 0.2) (layer "F.Cu") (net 21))
 (segment (start 113.7 105.6) (end 114.8125 104.4875) (width 0.2) (layer "F.Cu") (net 21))
 (segment (start 113.45 154.45) (end 113.8 154.1) (width 0.2) (layer "F.Cu") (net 21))
 (via (at 106.3 111.05) (size 0.6) (drill 0.3) (layers "F.Cu" "B.Cu") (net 21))
 (via (at 108.75 156.25) (size 0.6) (drill 0.3) (layers "F.Cu" "B.Cu") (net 21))
 (via (at 119.7 158.25) (size 0.6) (drill 0.3) (layers "F.Cu" "B.Cu") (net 21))
 (via (at 114.45 110.325) (size 0.6) (drill 0.3) (layers "F.Cu" "B.Cu") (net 21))
 (via (at 113.8 154.1) (size 0.6) (drill 0.3) (layers "F.Cu" "B.Cu") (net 21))
 (segment (start 114.45 111.7) (end 114.45 145.95) (width 0.2) (layer "B.Cu") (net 21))
 (segment (start 114.56 153.34) (end 113.8 154.1) (width 0.2) (layer "B.Cu") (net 21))
 (segment (start 110.9 154.1) (end 113.8 154.1) (width 0.2) (layer "B.Cu") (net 21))
 (segment (start 114.45 111.7) (end 114.45 110.325) (width 0.2) (layer "B.Cu") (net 21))
 (segment (start 113.025 113.125) (end 113.925 112.225) (width 0.2) (layer "B.Cu") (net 21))
 (segment (start 119.7 158.25) (end 119.7 155.35) (width 0.2) (layer "B.Cu") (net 21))
 (segment (start 113.925 112.225) (end 114.45 111.7) (width 0.2) (layer "B.Cu") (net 21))
 (segment (start 119.3 153.34) (end 119.3 150.8) (width 0.2) (layer "B.Cu") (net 21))
 (segment (start 119.3 153.34) (end 114.56 153.34) (width 0.2) (layer "B.Cu") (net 21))
 (segment (start 119.7 155.35) (end 119.3 154.95) (width 0.2) (layer "B.Cu") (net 21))
 (segment (start 119.3 154.95) (end 119.3 153.34) (width 0.2) (layer "B.Cu") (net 21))
 (segment (start 107.125 113.125) (end 106.3 112.3) (width 0.2) (layer "B.Cu") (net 21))
 (segment (start 114.45 145.95) (end 119.3 150.8) (width 0.2) (layer "B.Cu") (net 21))
 (segment (start 108.75 156.25) (end 110.9 154.1) (width 0.2) (layer "B.Cu") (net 21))
 (segment (start 106.3 112.3) (end 106.3 111.05) (width 0.2) (layer "B.Cu") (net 21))
 (segment (start 105.5 156.85) (end 105.8 156.85) (width 0.2) (layer "F.Cu") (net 22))
 (segment (start 103.25 158.75) (end 106.701 158.75) (width 0.2) (layer "F.Cu") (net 22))
 (segment (start 104.8 156.85) (end 105.5 156.85) (width 0.2) (layer "F.Cu") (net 22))
 (segment (start 113.95 159.002) (end 113.95 158.35) (width 0.2) (layer "F.Cu") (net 22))
 (segment (start 104.55 156.85) (end 104.58 156.85) (width 0.2) (layer "F.Cu") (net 22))
 (segment (start 106.701 158.75) (end 107.35 159.399) (width 0.2) (layer "F.Cu") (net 22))
 (segment (start 113.553 159.399) (end 113.95 159.002) (width 0.2) (layer "F.Cu") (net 22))
 (segment (start 111.151 158.9) (end 111.65 159.399) (width 0.2) (layer "F.Cu") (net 22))
 (segment (start 105.8 156.85) (end 107.85 158.9) (width 0.2) (layer "F.Cu") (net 22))
 (segment (start 110.399 159.399) (end 111.65 159.399) (width 0.2) (layer "F.Cu") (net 22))
 (segment (start 107.85 158.9) (end 111.151 158.9) (width 0.2) (layer "F.Cu") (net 22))
 (segment (start 111.65 159.399) (end 113.553 159.399) (width 0.2) (layer "F.Cu") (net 22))
 (segment (start 103.25 156.85) (end 104.55 156.85) (width 0.2) (layer "F.Cu") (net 22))
 (segment (start 107.35 159.399) (end 110.399 159.399) (width 0.2) (layer "F.Cu") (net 22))
 (segment (start 104.58 156.85) (end 105.5 155.93) (width 0.2) (layer "F.Cu") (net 22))
 (segment (start 104.55 156.85) (end 104.8 156.85) (width 0.2) (layer "F.Cu") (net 22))
 (segment (start 112.7 137.7) (end 112.7 156.1) (width 0.2) (layer "F.Cu") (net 3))
 (segment (start 97.4 107.78) (end 103 113.38) (width 0.2) (layer "F.Cu") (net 3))
 (segment (start 103 128) (end 112.7 137.7) (width 0.2) (layer "F.Cu") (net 3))
 (segment (start 103 113.38) (end 103 128) (width 0.2) (layer "F.Cu") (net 3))
 (segment (start 109.3 154.352) (end 109.3 151.65) (width 0.2) (layer "F.Cu") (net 17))
 (segment (start 102 144.35) (end 98.41 144.35) (width 0.2) (layer "F.Cu") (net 17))
 (segment (start 112.048 157.1) (end 109.3 154.352) (width 0.2) (layer "F.Cu") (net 17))
 (segment (start 98.41 144.35) (end 97.4 143.34) (width 0.2) (layer "F.Cu") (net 17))
 (segment (start 112.7 157.1) (end 112.048 157.1) (width 0.2) (layer "F.Cu") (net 17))
 (segment (start 109.3 151.65) (end 102 144.35) (width 0.2) (layer "F.Cu") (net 17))
 (segment (start 101.4 135.85) (end 101.4 114.32) (width 0.2) (layer "F.Cu") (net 4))
 (segment (start 110.9 145.35) (end 101.4 135.85) (width 0.2) (layer "F.Cu") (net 4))
 (segment (start 110.9 155.3849) (end 110.9 145.35) (width 0.2) (layer "F.Cu") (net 4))
 (segment (start 112.7 156.6) (end 112.1151 156.6) (width 0.2) (layer "F.Cu") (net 4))
 (segment (start 112.1151 156.6) (end 110.9 155.3849) (width 0.2) (layer "F.Cu") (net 4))
 (segment (start 101.4 114.32) (end 97.4 110.32) (width 0.2) (layer "F.Cu") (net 4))
 (segment (start 116.8 154.85) (end 116.25 154.3) (width 0.2) (layer "F.Cu") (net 25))
 (segment (start 116.25 154.3) (end 116.25 153.45) (width 0.2) (layer "F.Cu") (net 25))
 (segment (start 115 152.2) (end 115 128.15) (width 0.2) (layer "F.Cu") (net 25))
 (segment (start 115 128.15) (end 111.7 124.85) (width 0.2) (layer "F.Cu") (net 25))
 (segment (start 116.25 153.45) (end 115 152.2) (width 0.2) (layer "F.Cu") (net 25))
 (segment (start 115.7 156.6) (end 116.4 156.6) (width 0.2) (layer "F.Cu") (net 25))
 (segment (start 103.625 116.775) (end 103.625 113.275) (width 0.2) (layer "F.Cu") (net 25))
 (segment (start 106.075 119.225) (end 103.625 116.775) (width 0.2) (layer "F.Cu") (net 25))
 (segment (start 116.4 156.6) (end 116.8 156.2) (width 0.2) (layer "F.Cu") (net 25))
 (segment (start 111.7 124.85) (end 106.075 119.225) (width 0.2) (layer "F.Cu") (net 25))
 (segment (start 116.8 156.2) (end 116.8 154.85) (width 0.2) (layer "F.Cu") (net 25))
 (via (at 103.625 113.275) (size 0.6) (drill 0.3) (layers "F.Cu" "B.Cu") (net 25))
 (segment (start 104.2 113.275) (end 103.625 113.275) (width 0.2) (layer "B.Cu") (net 25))
 (segment (start 104.3 113.375) (end 104.2 113.275) (width 0.2) (layer "B.Cu") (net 25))
 (segment (start 115.7 157.6) (end 117 157.6) (width 0.2) (layer "F.Cu") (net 23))
 (segment (start 117.35 154.15) (end 117.35 152.85) (width 0.2) (layer "F.Cu") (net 23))
 (segment (start 105.2 116.75) (end 105.1 116.75) (width 0.2) (layer "F.Cu") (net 23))
 (segment (start 116.45 124.55) (end 112.75 120.85) (width 0.2) (layer "F.Cu") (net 23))
 (segment (start 106.2 116.75) (end 105.2 116.75) (width 0.2) (layer "F.Cu") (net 23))
 (segment (start 117 157.6) (end 117.8 156.8) (width 0.2) (layer "F.Cu") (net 23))
 (segment (start 117.8 154.6) (end 117.65 154.45) (width 0.2) (layer "F.Cu") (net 23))
 (segment (start 117.65 154.45) (end 117.35 154.15) (width 0.2) (layer "F.Cu") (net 23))
 (segment (start 116.45 151.95) (end 116.45 124.55) (width 0.2) (layer "F.Cu") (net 23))
 (segment (start 117.8 156.8) (end 117.8 154.6) (width 0.2) (layer "F.Cu") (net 23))
 (segment (start 112.75 120.85) (end 108.65 116.75) (width 0.2) (layer "F.Cu") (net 23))
 (segment (start 117.35 152.85) (end 116.45 151.95) (width 0.2) (layer "F.Cu") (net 23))
 (segment (start 108.65 116.75) (end 106.2 116.75) (width 0.2) (layer "F.Cu") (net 23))
 (via (at 105.2 116.75) (size 0.6) (drill 0.3) (layers "F.Cu" "B.Cu") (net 23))
 (segment (start 104.725 116.75) (end 104.15 116.175) (width 0.2) (layer "B.Cu") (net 23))
 (segment (start 104.15 116.175) (end 104.15 114.3) (width 0.2) (layer "B.Cu") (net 23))
 (segment (start 104.15 114.3) (end 104.375 114.075) (width 0.2) (layer "B.Cu") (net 23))
 (segment (start 105.2 116.75) (end 104.725 116.75) (width 0.2) (layer "B.Cu") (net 23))
 (segment (start 112.8 123.15) (end 107.7 118.05) (width 0.2) (layer "F.Cu") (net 24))
 (segment (start 115.75 152.1) (end 115.75 126.1) (width 0.2) (layer "F.Cu") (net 24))
 (segment (start 116.75 154.2) (end 116.75 153.1) (width 0.2) (layer "F.Cu") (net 24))
 (segment (start 116.75 153.1) (end 115.75 152.1) (width 0.2) (layer "F.Cu") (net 24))
 (segment (start 117.35 154.8) (end 116.75 154.2) (width 0.2) (layer "F.Cu") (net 24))
 (segment (start 117.35 156.55) (end 117.35 154.8) (width 0.2) (layer "F.Cu") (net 24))
 (segment (start 115.75 126.1) (end 112.8 123.15) (width 0.2) (layer "F.Cu") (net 24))
 (segment (start 115.7 157.1) (end 116.8 157.1) (width 0.2) (layer "F.Cu") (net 24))
 (segment (start 116.8 157.1) (end 117.35 156.55) (width 0.2) (layer "F.Cu") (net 24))
 (via (at 107.7 118.05) (size 0.6) (drill 0.3) (layers "F.Cu" "B.Cu") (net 24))
 (segment (start 105.9 113.1) (end 106.075 113.1) (width 0.2) (layer "B.Cu") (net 24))
 (segment (start 106.825 117.175) (end 107.7 118.05) (width 0.2) (layer "B.Cu") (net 24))
 (segment (start 106.825 113.85) (end 106.825 117.175) (width 0.2) (layer "B.Cu") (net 24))
 (segment (start 106.075 113.1) (end 106.825 113.85) (width 0.2) (layer "B.Cu") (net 24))
 (segment (start 114.3 151.1) (end 114.3 130.85) (width 0.2) (layer "F.Cu") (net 26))
 (segment (start 115.7 156.1) (end 115.7 153.95) (width 0.2) (layer "F.Cu") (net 26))
 (segment (start 111.5 128.05) (end 105.625 122.175) (width 0.2) (layer "F.Cu") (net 26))
 (segment (start 114.3 152.55) (end 114.3 151.1) (width 0.2) (layer "F.Cu") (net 26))
 (segment (start 105.625 122.175) (end 105.625 122.15) (width 0.2) (layer "F.Cu") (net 26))
 (segment (start 115.7 153.95) (end 114.3 152.55) (width 0.2) (layer "F.Cu") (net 26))
 (segment (start 114.3 130.85) (end 111.5 128.05) (width 0.2) (layer "F.Cu") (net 26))
 (via (at 105.625 122.15) (size 0.6) (drill 0.3) (layers "F.Cu" "B.Cu") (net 26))
 (segment (start 110.575 116.625) (end 110.575 114.825) (width 0.2) (layer "B.Cu") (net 26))
 (segment (start 105.625 121.575) (end 110.575 116.625) (width 0.2) (layer "B.Cu") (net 26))
 (segment (start 110.575 114.825) (end 111.075 114.325) (width 0.2) (layer "B.Cu") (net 26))
 (segment (start 105.625 122.15) (end 105.625 121.575) (width 0.2) (layer "B.Cu") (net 26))
 (segment (start 113.65 135.55) (end 106.6 128.5) (width 0.2) (layer "F.Cu") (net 27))
 (segment (start 113.65 151.2) (end 113.65 135.55) (width 0.2) (layer "F.Cu") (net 27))
 (segment (start 105.7 127.6) (end 105.7 125.05) (width 0.2) (layer "F.Cu") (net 27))
 (segment (start 106.6 128.5) (end 105.7 127.6) (width 0.2) (layer "F.Cu") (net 27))
 (segment (start 114.95 155.35) (end 114.95 154.2) (width 0.2) (layer "F.Cu") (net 27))
 (segment (start 114.95 154.2) (end 113.65 152.9) (width 0.2) (layer "F.Cu") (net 27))
 (segment (start 113.65 152.9) (end 113.65 151.2) (width 0.2) (layer "F.Cu") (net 27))
 (via (at 105.7 125.05) (size 0.6) (drill 0.3) (layers "F.Cu" "B.Cu") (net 27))
 (segment (start 105.7 124.2) (end 105.7 125.05) (width 0.2) (layer "B.Cu") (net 27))
 (segment (start 113.125 113.525) (end 113.575 113.975) (width 0.2) (layer "B.Cu") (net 27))
 (segment (start 113.05 113.525) (end 113.125 113.525) (width 0.2) (layer "B.Cu") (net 27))
 (segment (start 113.575 113.975) (end 113.575 116.325) (width 0.2) (layer "B.Cu") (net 27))
 (segment (start 113.575 116.325) (end 105.7 124.2) (width 0.2) (layer "B.Cu") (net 27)))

